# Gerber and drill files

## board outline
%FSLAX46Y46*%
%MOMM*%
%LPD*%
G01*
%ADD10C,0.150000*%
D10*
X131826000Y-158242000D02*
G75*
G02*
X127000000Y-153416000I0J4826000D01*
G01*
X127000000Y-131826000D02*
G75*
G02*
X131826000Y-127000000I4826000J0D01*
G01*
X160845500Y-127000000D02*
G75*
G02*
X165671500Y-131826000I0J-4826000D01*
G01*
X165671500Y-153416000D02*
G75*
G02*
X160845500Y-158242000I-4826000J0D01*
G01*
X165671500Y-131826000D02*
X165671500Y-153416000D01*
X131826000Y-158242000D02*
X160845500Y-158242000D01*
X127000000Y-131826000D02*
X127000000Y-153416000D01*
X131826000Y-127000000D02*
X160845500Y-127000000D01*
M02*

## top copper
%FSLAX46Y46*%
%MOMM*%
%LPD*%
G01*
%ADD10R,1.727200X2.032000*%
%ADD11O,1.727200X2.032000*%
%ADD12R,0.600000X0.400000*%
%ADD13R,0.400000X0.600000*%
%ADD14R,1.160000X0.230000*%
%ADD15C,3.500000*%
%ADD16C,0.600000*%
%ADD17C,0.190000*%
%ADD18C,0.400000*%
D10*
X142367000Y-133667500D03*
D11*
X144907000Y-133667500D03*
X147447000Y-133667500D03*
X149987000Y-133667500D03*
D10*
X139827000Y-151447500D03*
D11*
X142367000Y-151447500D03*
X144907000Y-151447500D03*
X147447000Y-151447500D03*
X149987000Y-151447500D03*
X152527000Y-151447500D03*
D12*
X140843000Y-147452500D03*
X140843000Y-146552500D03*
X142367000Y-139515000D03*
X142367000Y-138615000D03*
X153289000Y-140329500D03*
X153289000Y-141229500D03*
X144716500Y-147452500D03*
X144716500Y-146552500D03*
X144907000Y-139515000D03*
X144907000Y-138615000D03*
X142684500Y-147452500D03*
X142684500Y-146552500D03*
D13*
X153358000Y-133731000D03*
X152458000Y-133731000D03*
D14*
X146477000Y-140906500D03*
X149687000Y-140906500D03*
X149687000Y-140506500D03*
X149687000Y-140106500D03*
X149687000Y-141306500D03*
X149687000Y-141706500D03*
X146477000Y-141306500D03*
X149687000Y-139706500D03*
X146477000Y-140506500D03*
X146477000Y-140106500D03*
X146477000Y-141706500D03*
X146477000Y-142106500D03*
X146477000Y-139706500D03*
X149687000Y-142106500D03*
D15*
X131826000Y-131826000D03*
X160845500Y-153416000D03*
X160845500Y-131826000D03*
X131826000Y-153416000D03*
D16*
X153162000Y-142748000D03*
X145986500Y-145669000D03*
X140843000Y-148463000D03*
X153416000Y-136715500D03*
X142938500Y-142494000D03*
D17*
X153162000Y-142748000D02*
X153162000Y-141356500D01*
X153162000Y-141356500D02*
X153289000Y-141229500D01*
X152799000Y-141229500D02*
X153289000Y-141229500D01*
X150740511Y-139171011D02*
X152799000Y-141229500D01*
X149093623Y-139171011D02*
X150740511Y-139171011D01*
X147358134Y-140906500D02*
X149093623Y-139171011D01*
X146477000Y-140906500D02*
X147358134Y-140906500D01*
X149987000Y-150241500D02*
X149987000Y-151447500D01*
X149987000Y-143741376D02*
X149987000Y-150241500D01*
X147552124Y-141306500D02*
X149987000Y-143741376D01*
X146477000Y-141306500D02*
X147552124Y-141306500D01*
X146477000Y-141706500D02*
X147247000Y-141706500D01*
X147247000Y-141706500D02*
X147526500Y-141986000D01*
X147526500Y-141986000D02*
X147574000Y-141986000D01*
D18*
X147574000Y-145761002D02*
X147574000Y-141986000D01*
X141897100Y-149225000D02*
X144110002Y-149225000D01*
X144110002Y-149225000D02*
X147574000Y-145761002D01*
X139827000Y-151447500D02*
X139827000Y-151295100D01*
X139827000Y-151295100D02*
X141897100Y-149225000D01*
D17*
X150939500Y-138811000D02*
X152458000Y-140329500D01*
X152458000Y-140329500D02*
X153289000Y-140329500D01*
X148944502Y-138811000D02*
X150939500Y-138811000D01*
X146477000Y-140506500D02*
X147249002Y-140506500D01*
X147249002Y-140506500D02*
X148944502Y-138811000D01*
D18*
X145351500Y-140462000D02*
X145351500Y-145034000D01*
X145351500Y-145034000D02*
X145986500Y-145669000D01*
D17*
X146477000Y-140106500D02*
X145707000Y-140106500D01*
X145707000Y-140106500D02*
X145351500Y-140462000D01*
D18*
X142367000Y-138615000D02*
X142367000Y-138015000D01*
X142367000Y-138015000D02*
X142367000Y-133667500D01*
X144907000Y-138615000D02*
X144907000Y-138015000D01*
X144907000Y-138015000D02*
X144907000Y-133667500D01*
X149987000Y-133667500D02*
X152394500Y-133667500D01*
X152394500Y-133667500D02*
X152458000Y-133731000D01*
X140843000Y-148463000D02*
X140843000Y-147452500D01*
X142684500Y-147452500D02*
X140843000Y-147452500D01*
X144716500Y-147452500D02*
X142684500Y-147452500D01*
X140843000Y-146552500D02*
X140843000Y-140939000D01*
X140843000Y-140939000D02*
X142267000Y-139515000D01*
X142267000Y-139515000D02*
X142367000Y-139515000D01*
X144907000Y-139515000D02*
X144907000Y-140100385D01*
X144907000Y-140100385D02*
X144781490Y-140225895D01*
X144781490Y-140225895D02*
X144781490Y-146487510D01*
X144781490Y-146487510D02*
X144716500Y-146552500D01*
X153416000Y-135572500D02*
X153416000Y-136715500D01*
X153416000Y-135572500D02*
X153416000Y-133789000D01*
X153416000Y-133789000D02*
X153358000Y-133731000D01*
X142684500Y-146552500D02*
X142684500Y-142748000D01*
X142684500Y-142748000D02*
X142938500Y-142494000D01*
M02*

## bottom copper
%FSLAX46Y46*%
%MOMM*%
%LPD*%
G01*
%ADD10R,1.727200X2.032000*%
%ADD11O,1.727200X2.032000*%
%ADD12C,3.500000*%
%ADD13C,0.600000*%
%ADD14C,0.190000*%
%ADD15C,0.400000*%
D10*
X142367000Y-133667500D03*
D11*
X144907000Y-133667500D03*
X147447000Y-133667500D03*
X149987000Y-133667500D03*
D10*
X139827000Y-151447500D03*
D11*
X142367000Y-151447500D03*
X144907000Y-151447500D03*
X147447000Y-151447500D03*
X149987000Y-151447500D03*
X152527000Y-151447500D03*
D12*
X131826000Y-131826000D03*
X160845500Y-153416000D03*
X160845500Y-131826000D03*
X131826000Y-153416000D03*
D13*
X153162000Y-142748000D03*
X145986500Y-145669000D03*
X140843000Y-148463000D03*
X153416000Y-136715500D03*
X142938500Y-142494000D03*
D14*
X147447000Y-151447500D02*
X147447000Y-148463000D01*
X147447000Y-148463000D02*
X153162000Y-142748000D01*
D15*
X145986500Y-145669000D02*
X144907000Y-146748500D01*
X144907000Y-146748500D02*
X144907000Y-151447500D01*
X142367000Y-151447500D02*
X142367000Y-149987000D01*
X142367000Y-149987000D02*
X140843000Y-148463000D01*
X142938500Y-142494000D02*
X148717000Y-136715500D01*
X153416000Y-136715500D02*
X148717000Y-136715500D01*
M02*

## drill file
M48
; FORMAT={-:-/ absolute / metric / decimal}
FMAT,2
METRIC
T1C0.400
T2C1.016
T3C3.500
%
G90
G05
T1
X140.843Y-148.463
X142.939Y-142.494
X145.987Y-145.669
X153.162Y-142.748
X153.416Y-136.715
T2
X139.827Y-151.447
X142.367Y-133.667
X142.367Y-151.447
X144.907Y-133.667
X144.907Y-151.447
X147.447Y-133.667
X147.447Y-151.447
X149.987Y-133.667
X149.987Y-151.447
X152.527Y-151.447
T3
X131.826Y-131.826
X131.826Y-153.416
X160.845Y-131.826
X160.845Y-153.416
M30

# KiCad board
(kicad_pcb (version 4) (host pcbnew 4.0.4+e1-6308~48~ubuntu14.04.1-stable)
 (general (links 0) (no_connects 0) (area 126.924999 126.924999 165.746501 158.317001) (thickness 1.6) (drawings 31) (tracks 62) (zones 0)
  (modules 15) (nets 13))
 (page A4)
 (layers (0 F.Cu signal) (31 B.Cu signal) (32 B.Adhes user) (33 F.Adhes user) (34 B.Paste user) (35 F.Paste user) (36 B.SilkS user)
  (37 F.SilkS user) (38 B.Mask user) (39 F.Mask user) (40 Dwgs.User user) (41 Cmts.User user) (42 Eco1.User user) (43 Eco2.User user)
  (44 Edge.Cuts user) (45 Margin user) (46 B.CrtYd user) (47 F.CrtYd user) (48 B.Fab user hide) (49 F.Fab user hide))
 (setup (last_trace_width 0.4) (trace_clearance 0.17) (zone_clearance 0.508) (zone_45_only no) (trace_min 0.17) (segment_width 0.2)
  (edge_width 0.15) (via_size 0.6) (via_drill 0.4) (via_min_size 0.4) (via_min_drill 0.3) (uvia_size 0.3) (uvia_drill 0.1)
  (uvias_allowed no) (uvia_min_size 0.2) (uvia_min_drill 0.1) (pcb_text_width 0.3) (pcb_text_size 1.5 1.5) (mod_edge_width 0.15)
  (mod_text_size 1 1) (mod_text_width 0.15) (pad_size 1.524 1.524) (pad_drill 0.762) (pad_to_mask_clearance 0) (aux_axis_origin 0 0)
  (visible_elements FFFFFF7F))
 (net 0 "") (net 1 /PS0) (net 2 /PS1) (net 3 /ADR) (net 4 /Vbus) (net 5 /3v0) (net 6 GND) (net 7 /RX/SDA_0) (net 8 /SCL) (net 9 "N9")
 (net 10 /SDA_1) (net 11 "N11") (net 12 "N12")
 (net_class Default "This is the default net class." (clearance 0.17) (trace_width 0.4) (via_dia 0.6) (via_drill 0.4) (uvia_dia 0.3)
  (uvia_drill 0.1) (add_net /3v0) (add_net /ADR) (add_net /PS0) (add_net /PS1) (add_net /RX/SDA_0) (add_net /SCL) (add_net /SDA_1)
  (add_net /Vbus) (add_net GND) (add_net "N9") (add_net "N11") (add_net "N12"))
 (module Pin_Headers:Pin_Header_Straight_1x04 (layer F.Cu) (at 142.367 133.6675 90)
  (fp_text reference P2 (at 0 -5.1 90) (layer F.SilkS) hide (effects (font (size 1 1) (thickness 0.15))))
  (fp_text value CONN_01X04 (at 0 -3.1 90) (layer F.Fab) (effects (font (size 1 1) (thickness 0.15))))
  (pad 1 thru_hole rect (at 0 0 90) (size 2.032 1.7272) (drill 1.016) (layers *.Cu *.Mask) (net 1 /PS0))
  (pad 2 thru_hole oval (at 0 2.54 90) (size 2.032 1.7272) (drill 1.016) (layers *.Cu *.Mask) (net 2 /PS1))
  (pad 3 thru_hole oval (at 0 5.08 90) (size 2.032 1.7272) (drill 1.016) (layers *.Cu *.Mask))
  (pad 4 thru_hole oval (at 0 7.62 90) (size 2.032 1.7272) (drill 1.016) (layers *.Cu *.Mask) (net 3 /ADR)))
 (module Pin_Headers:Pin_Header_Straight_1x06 (layer F.Cu) (at 139.827 151.4475 90)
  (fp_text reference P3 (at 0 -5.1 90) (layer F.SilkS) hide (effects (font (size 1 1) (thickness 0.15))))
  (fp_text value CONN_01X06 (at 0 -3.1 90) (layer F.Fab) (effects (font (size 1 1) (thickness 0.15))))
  (pad 1 thru_hole rect (at 0 0 90) (size 2.032 1.7272) (drill 1.016) (layers *.Cu *.Mask) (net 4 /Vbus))
  (pad 2 thru_hole oval (at 0 2.54 90) (size 2.032 1.7272) (drill 1.016) (layers *.Cu *.Mask) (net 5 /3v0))
  (pad 3 thru_hole oval (at 0 5.08 90) (size 2.032 1.7272) (drill 1.016) (layers *.Cu *.Mask) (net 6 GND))
  (pad 4 thru_hole oval (at 0 7.62 90) (size 2.032 1.7272) (drill 1.016) (layers *.Cu *.Mask) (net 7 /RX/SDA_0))
  (pad 5 thru_hole oval (at 0 10.16 90) (size 2.032 1.7272) (drill 1.016) (layers *.Cu *.Mask) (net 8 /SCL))
  (pad 6 thru_hole oval (at 0 12.7 90) (size 2.032 1.7272) (drill 1.016) (layers *.Cu *.Mask)))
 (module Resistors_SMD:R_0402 (layer F.Cu) (at 140.843 147.0025 90)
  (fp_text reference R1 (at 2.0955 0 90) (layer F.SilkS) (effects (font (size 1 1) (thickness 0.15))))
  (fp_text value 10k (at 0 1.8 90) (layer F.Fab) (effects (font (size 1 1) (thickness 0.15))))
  (pad 1 smd rect (at -0.45 0 90) (size 0.4 0.6) (layers F.Cu F.Paste F.Mask) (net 5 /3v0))
  (pad 2 smd rect (at 0.45 0 90) (size 0.4 0.6) (layers F.Cu F.Paste F.Mask) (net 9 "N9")))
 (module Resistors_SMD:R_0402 (layer F.Cu) (at 142.367 139.065 90)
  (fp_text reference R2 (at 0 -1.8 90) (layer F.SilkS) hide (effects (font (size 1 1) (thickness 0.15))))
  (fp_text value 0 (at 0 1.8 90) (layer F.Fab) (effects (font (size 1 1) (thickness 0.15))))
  (pad 1 smd rect (at -0.45 0 90) (size 0.4 0.6) (layers F.Cu F.Paste F.Mask) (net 9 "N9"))
  (pad 2 smd rect (at 0.45 0 90) (size 0.4 0.6) (layers F.Cu F.Paste F.Mask) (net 1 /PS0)))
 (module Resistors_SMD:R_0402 (layer F.Cu) (at 153.289 140.7795 270)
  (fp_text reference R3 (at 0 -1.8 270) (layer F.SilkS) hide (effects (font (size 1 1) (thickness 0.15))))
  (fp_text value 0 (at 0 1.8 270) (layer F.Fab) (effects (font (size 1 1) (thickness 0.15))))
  (pad 1 smd rect (at -0.45 0 270) (size 0.4 0.6) (layers F.Cu F.Paste F.Mask) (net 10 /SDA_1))
  (pad 2 smd rect (at 0.45 0 270) (size 0.4 0.6) (layers F.Cu F.Paste F.Mask) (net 7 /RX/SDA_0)))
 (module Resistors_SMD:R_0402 (layer F.Cu) (at 144.7165 147.0025 90)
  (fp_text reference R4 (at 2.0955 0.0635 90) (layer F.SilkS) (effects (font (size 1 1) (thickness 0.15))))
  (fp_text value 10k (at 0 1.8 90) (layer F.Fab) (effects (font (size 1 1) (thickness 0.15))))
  (pad 1 smd rect (at -0.45 0 90) (size 0.4 0.6) (layers F.Cu F.Paste F.Mask) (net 5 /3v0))
  (pad 2 smd rect (at 0.45 0 90) (size 0.4 0.6) (layers F.Cu F.Paste F.Mask) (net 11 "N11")))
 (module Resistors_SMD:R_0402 (layer F.Cu) (at 144.907 139.065 90)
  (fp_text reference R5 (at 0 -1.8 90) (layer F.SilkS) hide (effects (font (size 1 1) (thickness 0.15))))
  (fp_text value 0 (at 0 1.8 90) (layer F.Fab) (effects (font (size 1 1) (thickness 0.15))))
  (pad 1 smd rect (at -0.45 0 90) (size 0.4 0.6) (layers F.Cu F.Paste F.Mask) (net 11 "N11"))
  (pad 2 smd rect (at 0.45 0 90) (size 0.4 0.6) (layers F.Cu F.Paste F.Mask) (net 2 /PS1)))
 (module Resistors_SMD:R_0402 (layer F.Cu) (at 142.6845 147.0025 90)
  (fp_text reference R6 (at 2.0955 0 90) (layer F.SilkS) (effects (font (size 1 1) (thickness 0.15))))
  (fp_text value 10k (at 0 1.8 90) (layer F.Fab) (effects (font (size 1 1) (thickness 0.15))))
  (pad 1 smd rect (at -0.45 0 90) (size 0.4 0.6) (layers F.Cu F.Paste F.Mask) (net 5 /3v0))
  (pad 2 smd rect (at 0.45 0 90) (size 0.4 0.6) (layers F.Cu F.Paste F.Mask) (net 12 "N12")))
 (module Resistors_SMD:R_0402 (layer F.Cu) (at 152.908 133.731 180)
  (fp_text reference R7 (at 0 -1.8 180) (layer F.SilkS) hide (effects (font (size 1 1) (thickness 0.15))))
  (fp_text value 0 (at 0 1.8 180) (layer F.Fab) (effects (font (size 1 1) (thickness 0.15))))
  (pad 1 smd rect (at -0.45 0 180) (size 0.4 0.6) (layers F.Cu F.Paste F.Mask) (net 12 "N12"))
  (pad 2 smd rect (at 0.45 0 180) (size 0.4 0.6) (layers F.Cu F.Paste F.Mask) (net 3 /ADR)))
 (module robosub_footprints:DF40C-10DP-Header (layer F.Cu) (at 148.082 140.9065 90)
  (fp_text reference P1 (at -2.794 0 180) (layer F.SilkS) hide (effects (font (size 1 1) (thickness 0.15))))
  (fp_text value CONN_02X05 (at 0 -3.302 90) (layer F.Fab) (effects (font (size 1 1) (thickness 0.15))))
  (pad 5 smd rect (at 0 -1.605 180) (size 1.16 0.23) (layers F.Cu F.Paste F.Mask) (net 7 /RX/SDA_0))
  (pad 6 smd rect (at 0 1.605 180) (size 1.16 0.23) (layers F.Cu F.Paste F.Mask))
  (pad 8 smd rect (at 0.4 1.605 180) (size 1.16 0.23) (layers F.Cu F.Paste F.Mask))
  (pad 10 smd rect (at 0.8 1.605 180) (size 1.16 0.23) (layers F.Cu F.Paste F.Mask))
  (pad 4 smd rect (at -0.4 1.605 180) (size 1.16 0.23) (layers F.Cu F.Paste F.Mask))
  (pad 2 smd rect (at -0.8 1.605 180) (size 1.16 0.23) (layers F.Cu F.Paste F.Mask))
  (pad 3 smd rect (at -0.4 -1.605 180) (size 1.16 0.23) (layers F.Cu F.Paste F.Mask) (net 8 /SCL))
  (pad ~ smd rect (at 1.2 1.605 180) (size 1.16 0.23) (layers F.Cu F.Paste F.Mask))
  (pad 7 smd rect (at 0.4 -1.605 180) (size 1.16 0.23) (layers F.Cu F.Paste F.Mask) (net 10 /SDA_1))
  (pad 9 smd rect (at 0.8 -1.605 180) (size 1.16 0.23) (layers F.Cu F.Paste F.Mask) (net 6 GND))
  (pad 1 smd rect (at -0.8 -1.605 180) (size 1.16 0.23) (layers F.Cu F.Paste F.Mask) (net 4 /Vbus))
  (pad ~ smd rect (at -1.2 -1.605 180) (size 1.16 0.23) (layers F.Cu F.Paste F.Mask))
  (pad ~ smd rect (at 1.2 -1.605 180) (size 1.16 0.23) (layers F.Cu F.Paste F.Mask))
  (pad ~ smd rect (at -1.2 1.605 180) (size 1.16 0.23) (layers F.Cu F.Paste F.Mask)))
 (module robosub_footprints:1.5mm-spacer (layer F.Cu) (at 131.826 131.826)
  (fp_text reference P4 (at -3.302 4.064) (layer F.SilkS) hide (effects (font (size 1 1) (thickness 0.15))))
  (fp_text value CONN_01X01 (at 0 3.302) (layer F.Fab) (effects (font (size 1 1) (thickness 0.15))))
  (pad "" thru_hole circle (at 0 0) (size 3.5 3.5) (drill 3.5) (layers *.Cu *.Mask F.SilkS)))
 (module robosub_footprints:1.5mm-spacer (layer F.Cu) (at 160.8455 153.416)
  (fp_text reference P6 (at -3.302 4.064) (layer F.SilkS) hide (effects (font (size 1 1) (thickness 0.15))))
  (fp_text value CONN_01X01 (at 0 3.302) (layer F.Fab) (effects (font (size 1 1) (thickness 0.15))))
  (pad "" thru_hole circle (at 0 0) (size 3.5 3.5) (drill 3.5) (layers *.Cu *.Mask F.SilkS)))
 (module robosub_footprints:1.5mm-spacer (layer F.Cu) (at 160.8455 131.826)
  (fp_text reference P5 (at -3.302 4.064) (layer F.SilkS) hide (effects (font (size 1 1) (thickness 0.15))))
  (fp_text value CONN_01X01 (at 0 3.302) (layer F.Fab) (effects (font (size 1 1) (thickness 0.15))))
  (pad "" thru_hole circle (at 0 0) (size 3.5 3.5) (drill 3.5) (layers *.Cu *.Mask F.SilkS)))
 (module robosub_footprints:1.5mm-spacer (layer F.Cu) (at 131.826 153.416)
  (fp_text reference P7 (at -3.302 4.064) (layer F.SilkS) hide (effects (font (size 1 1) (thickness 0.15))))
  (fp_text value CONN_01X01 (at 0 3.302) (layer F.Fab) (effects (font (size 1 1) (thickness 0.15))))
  (pad "" thru_hole circle (at 0 0) (size 3.5 3.5) (drill 3.5) (layers *.Cu *.Mask F.SilkS)))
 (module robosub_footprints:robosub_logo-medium (layer F.Cu) (at 130.048 142.8115 90)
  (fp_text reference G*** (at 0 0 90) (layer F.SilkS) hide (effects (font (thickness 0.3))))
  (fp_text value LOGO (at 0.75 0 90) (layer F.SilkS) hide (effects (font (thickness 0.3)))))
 (gr_arc (start 131.826 153.416) (end 131.826 158.242) (angle 90) (layer Edge.Cuts) (width 0.15))
 (gr_arc (start 131.826 131.826) (end 127 131.826) (angle 90) (layer Edge.Cuts) (width 0.15))
 (gr_arc (start 160.8455 131.826) (end 160.8455 127) (angle 90) (layer Edge.Cuts) (width 0.15))
 (gr_arc (start 160.8455 153.416) (end 165.6715 153.416) (angle 90) (layer Edge.Cuts) (width 0.15))
 (gr_line (start 165.6715 131.826) (end 165.6715 153.416) (layer Edge.Cuts) (width 0.15))
 (gr_line (start 131.826 158.242) (end 160.8455 158.242) (layer Edge.Cuts) (width 0.15))
 (gr_line (start 127 131.826) (end 127 153.416) (layer Edge.Cuts) (width 0.15))
 (gr_line (start 131.826 127) (end 160.8455 127) (layer Edge.Cuts) (width 0.15))
 (segment (start 153.162 142.748) (end 153.162 141.3565) (width 0.19) (layer F.Cu) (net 7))
 (segment (start 153.162 141.3565) (end 153.289 141.2295) (width 0.19) (layer F.Cu) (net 7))
 (segment (start 147.447 151.4475) (end 147.447 148.463) (width 0.19) (layer B.Cu) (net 7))
 (segment (start 147.447 148.463) (end 153.162 142.748) (width 0.19) (layer B.Cu) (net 7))
 (via (at 153.162 142.748) (size 0.6) (drill 0.4) (layers F.Cu B.Cu) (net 7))
 (segment (start 152.799 141.2295) (end 153.289 141.2295) (width 0.19) (layer F.Cu) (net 7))
 (segment (start 150.740511 139.171011) (end 152.799 141.2295) (width 0.19) (layer F.Cu) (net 7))
 (segment (start 149.093623 139.171011) (end 150.740511 139.171011) (width 0.19) (layer F.Cu) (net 7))
 (segment (start 147.358134 140.9065) (end 149.093623 139.171011) (width 0.19) (layer F.Cu) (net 7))
 (segment (start 146.477 140.9065) (end 147.358134 140.9065) (width 0.19) (layer F.Cu) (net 7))
 (segment (start 149.987 150.2415) (end 149.987 151.4475) (width 0.19) (layer F.Cu) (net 8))
 (segment (start 149.987 143.741376) (end 149.987 150.2415) (width 0.19) (layer F.Cu) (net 8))
 (segment (start 147.552124 141.3065) (end 149.987 143.741376) (width 0.19) (layer F.Cu) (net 8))
 (segment (start 146.477 141.3065) (end 147.552124 141.3065) (width 0.19) (layer F.Cu) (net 8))
 (segment (start 146.477 141.7065) (end 147.247 141.7065) (width 0.19) (layer F.Cu) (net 4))
 (segment (start 147.247 141.7065) (end 147.5265 141.986) (width 0.19) (layer F.Cu) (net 4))
 (segment (start 147.5265 141.986) (end 147.574 141.986) (width 0.19) (layer F.Cu) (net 4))
 (segment (start 147.574 145.761002) (end 147.574 141.986) (width 0.4) (layer F.Cu) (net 4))
 (segment (start 141.8971 149.225) (end 144.110002 149.225) (width 0.4) (layer F.Cu) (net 4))
 (segment (start 144.110002 149.225) (end 147.574 145.761002) (width 0.4) (layer F.Cu) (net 4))
 (segment (start 139.827 151.4475) (end 139.827 151.2951) (width 0.4) (layer F.Cu) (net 4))
 (segment (start 139.827 151.2951) (end 141.8971 149.225) (width 0.4) (layer F.Cu) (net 4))
 (segment (start 150.9395 138.811) (end 152.458 140.3295) (width 0.19) (layer F.Cu) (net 10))
 (segment (start 152.458 140.3295) (end 153.289 140.3295) (width 0.19) (layer F.Cu) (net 10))
 (segment (start 148.944502 138.811) (end 150.9395 138.811) (width 0.19) (layer F.Cu) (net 10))
 (segment (start 146.477 140.5065) (end 147.249002 140.5065) (width 0.19) (layer F.Cu) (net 10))
 (segment (start 147.249002 140.5065) (end 148.944502 138.811) (width 0.19) (layer F.Cu) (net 10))
 (segment (start 145.9865 145.669) (end 144.907 146.7485) (width 0.4) (layer B.Cu) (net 6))
 (segment (start 144.907 146.7485) (end 144.907 151.4475) (width 0.4) (layer B.Cu) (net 6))
 (segment (start 145.3515 140.462) (end 145.3515 145.034) (width 0.4) (layer F.Cu) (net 6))
 (segment (start 145.3515 145.034) (end 145.9865 145.669) (width 0.4) (layer F.Cu) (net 6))
 (via (at 145.9865 145.669) (size 0.6) (drill 0.4) (layers F.Cu B.Cu) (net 6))
 (segment (start 146.477 140.1065) (end 145.707 140.1065) (width 0.19) (layer F.Cu) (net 6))
 (segment (start 145.707 140.1065) (end 145.3515 140.462) (width 0.19) (layer F.Cu) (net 6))
 (segment (start 142.367 138.615) (end 142.367 138.015) (width 0.4) (layer F.Cu) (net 1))
 (segment (start 142.367 138.015) (end 142.367 133.6675) (width 0.4) (layer F.Cu) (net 1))
 (segment (start 144.907 138.615) (end 144.907 138.015) (width 0.4) (layer F.Cu) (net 2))
 (segment (start 144.907 138.015) (end 144.907 133.6675) (width 0.4) (layer F.Cu) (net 2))
 (segment (start 149.987 133.6675) (end 152.3945 133.6675) (width 0.4) (layer F.Cu) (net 3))
 (segment (start 152.3945 133.6675) (end 152.458 133.731) (width 0.4) (layer F.Cu) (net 3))
 (segment (start 140.843 148.463) (end 140.843 147.4525) (width 0.4) (layer F.Cu) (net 5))
 (segment (start 142.367 151.4475) (end 142.367 149.987) (width 0.4) (layer B.Cu) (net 5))
 (segment (start 142.367 149.987) (end 140.843 148.463) (width 0.4) (layer B.Cu) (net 5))
 (via (at 140.843 148.463) (size 0.6) (drill 0.4) (layers F.Cu B.Cu) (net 5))
 (segment (start 142.6845 147.4525) (end 140.843 147.4525) (width 0.4) (layer F.Cu) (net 5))
 (segment (start 144.7165 147.4525) (end 142.6845 147.4525) (width 0.4) (layer F.Cu) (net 5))
 (segment (start 140.843 146.5525) (end 140.843 140.939) (width 0.4) (layer F.Cu) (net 9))
 (segment (start 140.843 140.939) (end 142.267 139.515) (width 0.4) (layer F.Cu) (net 9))
 (segment (start 142.267 139.515) (end 142.367 139.515) (width 0.4) (layer F.Cu) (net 9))
 (segment (start 144.907 139.515) (end 144.907 140.100385) (width 0.4) (layer F.Cu) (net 11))
 (segment (start 144.907 140.100385) (end 144.78149 140.225895) (width 0.4) (layer F.Cu) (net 11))
 (segment (start 144.78149 140.225895) (end 144.78149 146.48751) (width 0.4) (layer F.Cu) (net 11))
 (segment (start 144.78149 146.48751) (end 144.7165 146.5525) (width 0.4) (layer F.Cu) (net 11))
 (segment (start 142.9385 142.494) (end 148.717 136.7155) (width 0.4) (layer B.Cu) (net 12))
 (segment (start 153.416 136.7155) (end 148.717 136.7155) (width 0.4) (layer B.Cu) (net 12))
 (segment (start 153.416 135.5725) (end 153.416 136.7155) (width 0.4) (layer F.Cu) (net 12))
 (via (at 153.416 136.7155) (size 0.6) (drill 0.4) (layers F.Cu B.Cu) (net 12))
 (segment (start 153.416 135.5725) (end 153.416 133.789) (width 0.4) (layer F.Cu) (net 12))
 (segment (start 153.416 133.789) (end 153.358 133.731) (width 0.4) (layer F.Cu) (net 12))
 (segment (start 142.6845 146.5525) (end 142.6845 142.748) (width 0.4) (layer F.Cu) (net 12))
 (segment (start 142.6845 142.748) (end 142.9385 142.494) (width 0.4) (layer F.Cu) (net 12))
 (via (at 142.9385 142.494) (size 0.6) (drill 0.4) (layers F.Cu B.Cu) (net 12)))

